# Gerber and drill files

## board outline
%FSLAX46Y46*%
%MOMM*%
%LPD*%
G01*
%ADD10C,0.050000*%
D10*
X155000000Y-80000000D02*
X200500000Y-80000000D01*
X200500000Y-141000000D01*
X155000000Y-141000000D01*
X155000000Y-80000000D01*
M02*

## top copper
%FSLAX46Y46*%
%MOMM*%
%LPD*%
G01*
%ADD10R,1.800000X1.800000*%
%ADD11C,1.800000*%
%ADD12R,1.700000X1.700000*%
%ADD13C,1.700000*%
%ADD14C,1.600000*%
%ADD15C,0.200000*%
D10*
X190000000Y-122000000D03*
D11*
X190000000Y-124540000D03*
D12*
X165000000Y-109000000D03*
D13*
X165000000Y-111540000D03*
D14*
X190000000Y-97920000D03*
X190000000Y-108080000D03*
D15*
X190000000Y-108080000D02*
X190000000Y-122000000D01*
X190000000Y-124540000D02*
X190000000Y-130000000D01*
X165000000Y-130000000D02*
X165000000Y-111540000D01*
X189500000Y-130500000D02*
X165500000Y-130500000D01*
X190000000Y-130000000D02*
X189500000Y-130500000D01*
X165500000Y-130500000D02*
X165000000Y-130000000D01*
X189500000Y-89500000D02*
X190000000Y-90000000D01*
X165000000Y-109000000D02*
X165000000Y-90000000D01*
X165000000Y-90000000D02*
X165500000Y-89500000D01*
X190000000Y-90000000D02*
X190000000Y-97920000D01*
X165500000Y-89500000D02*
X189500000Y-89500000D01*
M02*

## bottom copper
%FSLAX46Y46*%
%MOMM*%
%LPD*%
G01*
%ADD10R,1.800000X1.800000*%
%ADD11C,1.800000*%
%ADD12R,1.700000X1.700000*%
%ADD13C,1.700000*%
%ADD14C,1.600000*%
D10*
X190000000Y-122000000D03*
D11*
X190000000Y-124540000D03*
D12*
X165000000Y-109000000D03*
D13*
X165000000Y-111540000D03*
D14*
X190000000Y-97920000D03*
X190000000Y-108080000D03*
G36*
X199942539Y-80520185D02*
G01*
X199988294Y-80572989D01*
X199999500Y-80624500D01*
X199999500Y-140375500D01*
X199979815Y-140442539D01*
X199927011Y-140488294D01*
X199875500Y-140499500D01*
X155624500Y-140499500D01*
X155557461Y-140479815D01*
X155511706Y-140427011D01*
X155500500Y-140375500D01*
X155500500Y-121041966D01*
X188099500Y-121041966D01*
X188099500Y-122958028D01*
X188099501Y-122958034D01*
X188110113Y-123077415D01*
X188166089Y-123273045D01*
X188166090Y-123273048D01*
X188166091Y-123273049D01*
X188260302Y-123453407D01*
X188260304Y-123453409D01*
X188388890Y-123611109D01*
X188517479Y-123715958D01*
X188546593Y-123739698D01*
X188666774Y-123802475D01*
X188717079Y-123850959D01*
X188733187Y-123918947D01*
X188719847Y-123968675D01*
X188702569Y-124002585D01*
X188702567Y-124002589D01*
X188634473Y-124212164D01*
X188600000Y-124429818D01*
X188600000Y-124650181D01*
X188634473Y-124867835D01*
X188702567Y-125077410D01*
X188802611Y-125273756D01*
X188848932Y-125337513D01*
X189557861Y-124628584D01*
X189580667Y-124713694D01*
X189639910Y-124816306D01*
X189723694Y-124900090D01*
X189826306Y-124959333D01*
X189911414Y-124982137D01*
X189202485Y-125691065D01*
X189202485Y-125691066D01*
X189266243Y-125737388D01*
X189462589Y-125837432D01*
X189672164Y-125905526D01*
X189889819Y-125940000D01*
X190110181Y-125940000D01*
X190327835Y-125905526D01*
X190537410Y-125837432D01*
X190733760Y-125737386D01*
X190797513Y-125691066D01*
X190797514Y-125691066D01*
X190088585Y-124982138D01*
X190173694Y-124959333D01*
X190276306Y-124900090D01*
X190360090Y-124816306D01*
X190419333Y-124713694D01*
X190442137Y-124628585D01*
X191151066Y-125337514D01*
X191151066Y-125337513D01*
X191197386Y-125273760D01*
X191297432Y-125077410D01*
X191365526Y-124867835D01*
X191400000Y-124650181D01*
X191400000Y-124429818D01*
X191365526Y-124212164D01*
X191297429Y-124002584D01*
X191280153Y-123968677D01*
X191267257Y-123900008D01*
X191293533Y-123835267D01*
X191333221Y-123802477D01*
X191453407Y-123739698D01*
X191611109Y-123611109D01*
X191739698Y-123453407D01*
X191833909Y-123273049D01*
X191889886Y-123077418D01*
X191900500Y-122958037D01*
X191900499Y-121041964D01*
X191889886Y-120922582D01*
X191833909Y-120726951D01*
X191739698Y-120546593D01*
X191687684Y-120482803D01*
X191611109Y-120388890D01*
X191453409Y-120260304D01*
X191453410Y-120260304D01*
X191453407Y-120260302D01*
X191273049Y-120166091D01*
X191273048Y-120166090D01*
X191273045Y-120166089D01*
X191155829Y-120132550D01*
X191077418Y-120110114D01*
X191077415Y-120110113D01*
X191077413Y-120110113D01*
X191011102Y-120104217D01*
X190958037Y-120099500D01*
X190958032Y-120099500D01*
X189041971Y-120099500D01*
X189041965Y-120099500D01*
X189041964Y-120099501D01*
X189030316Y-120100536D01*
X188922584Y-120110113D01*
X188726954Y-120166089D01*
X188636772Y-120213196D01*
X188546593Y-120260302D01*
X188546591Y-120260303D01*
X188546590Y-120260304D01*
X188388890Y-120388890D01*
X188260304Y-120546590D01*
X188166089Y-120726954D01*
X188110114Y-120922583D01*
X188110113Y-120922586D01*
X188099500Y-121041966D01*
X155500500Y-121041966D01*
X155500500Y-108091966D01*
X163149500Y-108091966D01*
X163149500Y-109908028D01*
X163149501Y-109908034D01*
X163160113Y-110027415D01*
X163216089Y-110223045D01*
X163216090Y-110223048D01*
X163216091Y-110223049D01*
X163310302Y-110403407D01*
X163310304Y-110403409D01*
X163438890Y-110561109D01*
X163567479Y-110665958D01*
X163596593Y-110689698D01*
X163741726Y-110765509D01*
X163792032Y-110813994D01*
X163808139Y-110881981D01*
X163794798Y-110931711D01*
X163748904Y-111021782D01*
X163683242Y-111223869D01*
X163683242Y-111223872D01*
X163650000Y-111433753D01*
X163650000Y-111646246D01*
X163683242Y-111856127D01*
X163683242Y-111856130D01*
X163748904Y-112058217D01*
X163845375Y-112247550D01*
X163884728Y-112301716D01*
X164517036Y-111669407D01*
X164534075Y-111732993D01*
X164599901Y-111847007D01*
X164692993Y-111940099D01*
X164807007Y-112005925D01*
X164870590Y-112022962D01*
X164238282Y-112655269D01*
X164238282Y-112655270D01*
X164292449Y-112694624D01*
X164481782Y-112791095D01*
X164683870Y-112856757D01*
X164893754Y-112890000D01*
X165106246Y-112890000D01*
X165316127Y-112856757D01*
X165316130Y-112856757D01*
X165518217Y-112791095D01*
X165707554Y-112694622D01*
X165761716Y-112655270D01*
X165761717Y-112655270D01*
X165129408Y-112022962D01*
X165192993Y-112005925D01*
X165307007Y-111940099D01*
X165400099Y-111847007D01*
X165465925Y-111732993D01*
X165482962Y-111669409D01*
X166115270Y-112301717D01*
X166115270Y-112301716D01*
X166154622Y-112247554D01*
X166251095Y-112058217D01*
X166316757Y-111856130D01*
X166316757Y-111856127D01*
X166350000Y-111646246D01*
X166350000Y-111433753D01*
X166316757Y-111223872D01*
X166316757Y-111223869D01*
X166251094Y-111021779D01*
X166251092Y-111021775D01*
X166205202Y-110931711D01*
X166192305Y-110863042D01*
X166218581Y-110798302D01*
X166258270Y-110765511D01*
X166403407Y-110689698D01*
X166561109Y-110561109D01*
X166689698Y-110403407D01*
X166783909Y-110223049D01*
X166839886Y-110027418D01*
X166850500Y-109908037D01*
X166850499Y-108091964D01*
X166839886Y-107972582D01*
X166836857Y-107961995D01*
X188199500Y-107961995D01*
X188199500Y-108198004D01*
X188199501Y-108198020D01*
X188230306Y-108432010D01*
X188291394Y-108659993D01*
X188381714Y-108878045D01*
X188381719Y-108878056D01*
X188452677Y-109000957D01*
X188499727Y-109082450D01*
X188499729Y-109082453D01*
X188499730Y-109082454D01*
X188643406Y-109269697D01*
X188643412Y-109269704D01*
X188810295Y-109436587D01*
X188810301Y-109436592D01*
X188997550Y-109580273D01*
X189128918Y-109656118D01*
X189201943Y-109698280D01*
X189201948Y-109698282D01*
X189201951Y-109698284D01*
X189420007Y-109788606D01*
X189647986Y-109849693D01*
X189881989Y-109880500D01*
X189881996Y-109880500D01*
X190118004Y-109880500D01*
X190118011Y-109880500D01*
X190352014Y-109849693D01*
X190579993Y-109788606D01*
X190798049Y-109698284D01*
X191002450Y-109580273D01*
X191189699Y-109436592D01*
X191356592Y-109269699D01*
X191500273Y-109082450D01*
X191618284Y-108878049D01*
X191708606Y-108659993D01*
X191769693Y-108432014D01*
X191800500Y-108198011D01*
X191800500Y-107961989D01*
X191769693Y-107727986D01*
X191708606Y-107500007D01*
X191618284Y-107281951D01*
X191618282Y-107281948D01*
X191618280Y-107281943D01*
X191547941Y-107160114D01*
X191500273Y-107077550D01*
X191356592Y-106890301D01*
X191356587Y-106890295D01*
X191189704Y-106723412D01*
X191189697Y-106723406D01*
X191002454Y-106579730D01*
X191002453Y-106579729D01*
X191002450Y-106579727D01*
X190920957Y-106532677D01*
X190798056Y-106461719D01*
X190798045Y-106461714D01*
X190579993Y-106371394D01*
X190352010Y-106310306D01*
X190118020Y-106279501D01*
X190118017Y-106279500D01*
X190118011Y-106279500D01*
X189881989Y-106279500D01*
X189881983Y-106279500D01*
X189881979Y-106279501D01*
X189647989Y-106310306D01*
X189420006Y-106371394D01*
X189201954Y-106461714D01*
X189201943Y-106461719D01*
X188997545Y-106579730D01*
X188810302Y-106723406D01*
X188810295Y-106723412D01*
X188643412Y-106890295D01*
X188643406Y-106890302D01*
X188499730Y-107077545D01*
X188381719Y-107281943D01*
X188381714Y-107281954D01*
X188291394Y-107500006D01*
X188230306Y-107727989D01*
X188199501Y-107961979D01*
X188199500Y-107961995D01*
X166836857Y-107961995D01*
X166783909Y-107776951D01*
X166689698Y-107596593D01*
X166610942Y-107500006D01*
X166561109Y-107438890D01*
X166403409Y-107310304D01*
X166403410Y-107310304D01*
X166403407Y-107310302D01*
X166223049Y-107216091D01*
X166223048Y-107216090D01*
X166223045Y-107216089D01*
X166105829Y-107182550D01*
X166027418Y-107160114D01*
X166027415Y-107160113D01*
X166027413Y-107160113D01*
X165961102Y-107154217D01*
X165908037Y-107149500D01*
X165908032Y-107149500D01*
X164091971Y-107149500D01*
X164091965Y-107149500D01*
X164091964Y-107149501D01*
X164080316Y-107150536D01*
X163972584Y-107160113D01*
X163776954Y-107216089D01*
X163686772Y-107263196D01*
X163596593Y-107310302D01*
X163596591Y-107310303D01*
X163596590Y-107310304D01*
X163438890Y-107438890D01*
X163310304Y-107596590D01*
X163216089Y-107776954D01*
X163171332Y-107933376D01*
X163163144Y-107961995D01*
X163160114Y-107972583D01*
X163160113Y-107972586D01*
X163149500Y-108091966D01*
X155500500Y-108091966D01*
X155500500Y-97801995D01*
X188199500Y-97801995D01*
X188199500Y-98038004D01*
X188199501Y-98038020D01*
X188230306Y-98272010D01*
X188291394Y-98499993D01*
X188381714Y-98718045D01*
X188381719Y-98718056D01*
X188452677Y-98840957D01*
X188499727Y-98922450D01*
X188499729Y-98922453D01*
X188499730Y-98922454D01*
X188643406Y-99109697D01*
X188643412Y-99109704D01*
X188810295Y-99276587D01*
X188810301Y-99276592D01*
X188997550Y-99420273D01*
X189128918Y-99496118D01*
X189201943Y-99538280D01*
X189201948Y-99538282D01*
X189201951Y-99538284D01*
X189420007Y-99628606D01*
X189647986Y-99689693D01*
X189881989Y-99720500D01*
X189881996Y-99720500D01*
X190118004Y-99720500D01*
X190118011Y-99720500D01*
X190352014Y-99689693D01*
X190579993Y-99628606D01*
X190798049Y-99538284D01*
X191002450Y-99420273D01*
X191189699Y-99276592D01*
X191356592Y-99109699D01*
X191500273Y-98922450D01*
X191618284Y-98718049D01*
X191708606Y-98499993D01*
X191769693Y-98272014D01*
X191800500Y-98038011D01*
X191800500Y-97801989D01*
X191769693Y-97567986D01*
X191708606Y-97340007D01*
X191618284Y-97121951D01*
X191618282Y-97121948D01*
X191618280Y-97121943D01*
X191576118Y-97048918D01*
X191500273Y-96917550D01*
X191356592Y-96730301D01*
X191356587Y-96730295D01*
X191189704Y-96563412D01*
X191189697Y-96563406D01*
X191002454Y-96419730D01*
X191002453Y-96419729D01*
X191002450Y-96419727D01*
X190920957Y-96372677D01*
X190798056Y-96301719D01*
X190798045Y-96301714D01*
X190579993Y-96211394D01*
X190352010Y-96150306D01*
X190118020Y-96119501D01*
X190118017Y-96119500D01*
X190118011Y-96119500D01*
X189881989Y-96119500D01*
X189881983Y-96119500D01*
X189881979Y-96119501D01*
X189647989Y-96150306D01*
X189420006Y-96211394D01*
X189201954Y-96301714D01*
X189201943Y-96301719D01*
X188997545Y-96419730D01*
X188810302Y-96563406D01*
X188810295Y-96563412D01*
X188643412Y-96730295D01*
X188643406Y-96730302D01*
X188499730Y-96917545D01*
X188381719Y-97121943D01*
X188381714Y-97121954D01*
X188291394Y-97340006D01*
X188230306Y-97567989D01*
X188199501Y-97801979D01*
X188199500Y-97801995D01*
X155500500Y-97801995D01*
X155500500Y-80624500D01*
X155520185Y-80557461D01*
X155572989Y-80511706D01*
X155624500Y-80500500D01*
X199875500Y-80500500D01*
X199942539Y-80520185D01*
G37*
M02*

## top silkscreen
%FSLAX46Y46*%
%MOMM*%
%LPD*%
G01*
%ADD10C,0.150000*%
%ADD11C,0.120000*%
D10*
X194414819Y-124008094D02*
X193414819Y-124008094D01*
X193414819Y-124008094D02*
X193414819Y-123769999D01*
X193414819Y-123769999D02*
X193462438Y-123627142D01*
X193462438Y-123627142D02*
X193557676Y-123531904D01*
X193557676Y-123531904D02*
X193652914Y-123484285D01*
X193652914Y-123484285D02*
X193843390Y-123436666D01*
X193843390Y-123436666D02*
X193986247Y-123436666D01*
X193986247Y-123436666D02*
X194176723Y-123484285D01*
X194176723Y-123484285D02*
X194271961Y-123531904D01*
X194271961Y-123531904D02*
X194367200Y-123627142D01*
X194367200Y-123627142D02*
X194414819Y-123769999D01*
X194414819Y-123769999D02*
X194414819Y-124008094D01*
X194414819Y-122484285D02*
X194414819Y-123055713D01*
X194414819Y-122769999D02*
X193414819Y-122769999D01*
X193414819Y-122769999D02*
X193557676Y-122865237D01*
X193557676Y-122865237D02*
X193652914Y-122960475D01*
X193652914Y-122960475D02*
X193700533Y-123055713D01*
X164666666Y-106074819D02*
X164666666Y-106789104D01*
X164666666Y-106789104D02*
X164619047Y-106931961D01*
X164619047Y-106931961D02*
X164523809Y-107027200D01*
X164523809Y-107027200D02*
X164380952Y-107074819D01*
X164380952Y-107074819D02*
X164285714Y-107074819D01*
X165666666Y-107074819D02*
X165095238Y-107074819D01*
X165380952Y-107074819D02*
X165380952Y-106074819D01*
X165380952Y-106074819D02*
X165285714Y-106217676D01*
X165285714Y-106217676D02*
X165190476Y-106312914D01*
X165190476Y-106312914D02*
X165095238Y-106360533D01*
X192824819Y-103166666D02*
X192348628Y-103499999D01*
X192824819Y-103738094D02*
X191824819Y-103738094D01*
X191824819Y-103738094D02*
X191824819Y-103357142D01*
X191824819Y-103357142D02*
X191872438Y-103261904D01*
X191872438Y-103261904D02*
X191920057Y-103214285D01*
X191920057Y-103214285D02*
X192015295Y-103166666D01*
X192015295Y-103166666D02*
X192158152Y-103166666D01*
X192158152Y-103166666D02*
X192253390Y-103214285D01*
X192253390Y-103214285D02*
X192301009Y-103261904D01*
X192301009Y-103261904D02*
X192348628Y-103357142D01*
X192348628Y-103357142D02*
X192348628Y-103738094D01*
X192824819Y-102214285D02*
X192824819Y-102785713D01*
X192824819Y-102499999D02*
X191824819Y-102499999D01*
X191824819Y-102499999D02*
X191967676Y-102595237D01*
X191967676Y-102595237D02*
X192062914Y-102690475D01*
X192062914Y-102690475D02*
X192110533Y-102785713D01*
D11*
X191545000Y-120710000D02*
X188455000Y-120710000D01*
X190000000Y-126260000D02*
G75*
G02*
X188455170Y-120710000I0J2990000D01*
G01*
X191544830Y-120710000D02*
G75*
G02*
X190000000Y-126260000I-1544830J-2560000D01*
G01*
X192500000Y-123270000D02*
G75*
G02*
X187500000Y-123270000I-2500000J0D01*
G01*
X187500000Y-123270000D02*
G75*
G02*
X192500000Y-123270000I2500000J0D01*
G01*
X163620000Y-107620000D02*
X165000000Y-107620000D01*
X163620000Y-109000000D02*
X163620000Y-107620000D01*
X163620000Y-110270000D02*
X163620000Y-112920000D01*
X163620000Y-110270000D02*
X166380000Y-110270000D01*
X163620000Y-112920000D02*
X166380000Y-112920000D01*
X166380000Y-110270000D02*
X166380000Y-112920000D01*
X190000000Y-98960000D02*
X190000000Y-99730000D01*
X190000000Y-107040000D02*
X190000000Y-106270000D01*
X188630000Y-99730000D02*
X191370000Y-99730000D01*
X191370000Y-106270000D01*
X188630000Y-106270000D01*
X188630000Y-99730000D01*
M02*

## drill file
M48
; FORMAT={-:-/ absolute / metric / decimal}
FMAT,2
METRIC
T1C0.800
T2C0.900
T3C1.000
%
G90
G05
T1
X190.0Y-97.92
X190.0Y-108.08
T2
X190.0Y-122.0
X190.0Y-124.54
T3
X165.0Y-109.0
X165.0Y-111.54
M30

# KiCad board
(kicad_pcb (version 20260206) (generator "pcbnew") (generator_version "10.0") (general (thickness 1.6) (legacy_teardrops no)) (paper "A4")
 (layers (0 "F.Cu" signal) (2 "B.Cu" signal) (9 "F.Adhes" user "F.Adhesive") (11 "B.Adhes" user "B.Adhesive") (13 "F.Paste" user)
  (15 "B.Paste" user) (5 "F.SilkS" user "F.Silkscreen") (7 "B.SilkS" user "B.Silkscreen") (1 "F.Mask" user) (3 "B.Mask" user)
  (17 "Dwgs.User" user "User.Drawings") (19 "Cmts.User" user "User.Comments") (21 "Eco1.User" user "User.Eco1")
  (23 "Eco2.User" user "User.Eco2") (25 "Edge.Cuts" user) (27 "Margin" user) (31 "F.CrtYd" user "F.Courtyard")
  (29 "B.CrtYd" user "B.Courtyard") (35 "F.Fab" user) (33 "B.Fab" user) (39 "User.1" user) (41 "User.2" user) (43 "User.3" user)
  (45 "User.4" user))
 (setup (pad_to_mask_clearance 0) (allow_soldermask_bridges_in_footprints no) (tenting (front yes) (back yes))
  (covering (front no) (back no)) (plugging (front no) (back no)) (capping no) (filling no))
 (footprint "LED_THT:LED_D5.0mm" (layer "F.Cu") (at 190 122 -90)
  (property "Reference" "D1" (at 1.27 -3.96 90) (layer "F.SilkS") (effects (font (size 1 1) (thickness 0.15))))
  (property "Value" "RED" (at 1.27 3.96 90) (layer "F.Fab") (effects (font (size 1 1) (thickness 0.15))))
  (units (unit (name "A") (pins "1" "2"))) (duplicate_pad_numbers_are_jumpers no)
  (fp_line (start -1.29 -1.545) (end -1.29 1.545) (stroke (width 0.12) (type solid)) (layer "F.SilkS"))
  (fp_arc (start 4.26 0) (mid 2.071779 2.880495) (end -1.29 1.54483) (stroke (width 0.12) (type solid)) (layer "F.SilkS"))
  (fp_arc (start -1.29 -1.54483) (mid 2.071779 -2.880495) (end 4.26 0) (stroke (width 0.12) (type solid)) (layer "F.SilkS"))
  (fp_circle (center 1.27 0) (end 3.77 0) (stroke (width 0.12) (type solid)) (fill no) (layer "F.SilkS"))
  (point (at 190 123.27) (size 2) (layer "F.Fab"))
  (pad "1" thru_hole rect (at 0 0 270) (size 1.8 1.8) (drill 0.9) (layers "*.Cu" "*.Mask") (remove_unused_layers no) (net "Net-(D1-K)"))
  (pad "2" thru_hole circle (at 2.54 0 270) (size 1.8 1.8) (drill 0.9) (layers "*.Cu" "*.Mask") (remove_unused_layers no) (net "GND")))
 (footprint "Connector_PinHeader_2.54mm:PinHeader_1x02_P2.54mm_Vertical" (layer "F.Cu") (at 165 109)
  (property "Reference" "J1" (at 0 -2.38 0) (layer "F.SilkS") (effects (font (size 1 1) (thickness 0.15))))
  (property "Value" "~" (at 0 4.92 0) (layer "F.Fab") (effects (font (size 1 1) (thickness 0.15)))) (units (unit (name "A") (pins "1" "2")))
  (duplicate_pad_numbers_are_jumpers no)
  (fp_line (start -1.38 -1.38) (end 0 -1.38) (stroke (width 0.12) (type solid)) (layer "F.SilkS"))
  (fp_line (start -1.38 0) (end -1.38 -1.38) (stroke (width 0.12) (type solid)) (layer "F.SilkS"))
  (fp_line (start -1.38 1.27) (end -1.38 3.92) (stroke (width 0.12) (type solid)) (layer "F.SilkS"))
  (fp_line (start -1.38 1.27) (end 1.38 1.27) (stroke (width 0.12) (type solid)) (layer "F.SilkS"))
  (fp_line (start -1.38 3.92) (end 1.38 3.92) (stroke (width 0.12) (type solid)) (layer "F.SilkS"))
  (fp_line (start 1.38 1.27) (end 1.38 3.92) (stroke (width 0.12) (type solid)) (layer "F.SilkS"))
  (pad "1" thru_hole rect (at 0 0) (size 1.7 1.7) (drill 1) (layers "*.Cu" "*.Mask") (remove_unused_layers no) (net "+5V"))
  (pad "2" thru_hole circle (at 0 2.54) (size 1.7 1.7) (drill 1) (layers "*.Cu" "*.Mask") (remove_unused_layers no) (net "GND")))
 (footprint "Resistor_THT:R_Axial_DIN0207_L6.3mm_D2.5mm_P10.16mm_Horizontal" (layer "F.Cu") (at 190 97.92 -90)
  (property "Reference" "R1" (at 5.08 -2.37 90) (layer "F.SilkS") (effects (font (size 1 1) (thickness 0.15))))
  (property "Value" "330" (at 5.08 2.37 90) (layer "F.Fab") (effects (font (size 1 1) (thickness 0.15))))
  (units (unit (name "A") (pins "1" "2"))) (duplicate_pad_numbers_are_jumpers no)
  (fp_line (start 1.04 0) (end 1.81 0) (stroke (width 0.12) (type solid)) (layer "F.SilkS"))
  (fp_line (start 9.12 0) (end 8.35 0) (stroke (width 0.12) (type solid)) (layer "F.SilkS"))
  (fp_rect (start 1.81 -1.37) (end 8.35 1.37) (stroke (width 0.12) (type solid)) (fill no) (layer "F.SilkS"))
  (pad "1" thru_hole circle (at 0 0 270) (size 1.6 1.6) (drill 0.8) (layers "*.Cu" "*.Mask") (remove_unused_layers no) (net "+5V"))
  (pad "2" thru_hole circle (at 10.16 0 270) (size 1.6 1.6) (drill 0.8) (layers "*.Cu" "*.Mask") (remove_unused_layers no)
   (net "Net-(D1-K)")))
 (gr_rect (start 155 80) (end 200.5 141) (stroke (width 0.05) (type default)) (fill no) (layer "Edge.Cuts"))
 (segment (start 190 108.08) (end 190 122) (width 0.2) (layers "F.Cu" "F.Mask") (solder_mask_margin 0.2) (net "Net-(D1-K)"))
 (segment (start 190 124.54) (end 190 130) (width 0.2) (layers "F.Cu" "F.Mask") (solder_mask_margin 0.2) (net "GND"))
 (segment (start 165 130) (end 165 111.54) (width 0.2) (layers "F.Cu" "F.Mask") (solder_mask_margin 0.2) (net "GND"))
 (segment (start 189.5 130.5) (end 165.5 130.5) (width 0.2) (layers "F.Cu" "F.Mask") (solder_mask_margin 0.2) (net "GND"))
 (segment (start 190 130) (end 189.5 130.5) (width 0.2) (layers "F.Cu" "F.Mask") (solder_mask_margin 0.2) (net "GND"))
 (segment (start 165.5 130.5) (end 165 130) (width 0.2) (layers "F.Cu" "F.Mask") (solder_mask_margin 0.2) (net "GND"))
 (segment (start 189.5 89.5) (end 190 90) (width 0.2) (layers "F.Cu" "F.Mask") (solder_mask_margin 0.2) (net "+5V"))
 (segment (start 165 109) (end 165 90) (width 0.2) (layers "F.Cu" "F.Mask") (solder_mask_margin 0.2) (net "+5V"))
 (segment (start 165 90) (end 165.5 89.5) (width 0.2) (layers "F.Cu" "F.Mask") (solder_mask_margin 0.2) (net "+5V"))
 (segment (start 190 90) (end 190 97.92) (width 0.2) (layers "F.Cu" "F.Mask") (solder_mask_margin 0.2) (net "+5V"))
 (segment (start 165.5 89.5) (end 189.5 89.5) (width 0.2) (layers "F.Cu" "F.Mask") (solder_mask_margin 0.2) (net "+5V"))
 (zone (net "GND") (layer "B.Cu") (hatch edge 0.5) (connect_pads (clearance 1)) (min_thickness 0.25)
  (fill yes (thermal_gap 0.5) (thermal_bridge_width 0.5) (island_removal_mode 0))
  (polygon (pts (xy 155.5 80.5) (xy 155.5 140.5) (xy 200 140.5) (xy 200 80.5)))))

